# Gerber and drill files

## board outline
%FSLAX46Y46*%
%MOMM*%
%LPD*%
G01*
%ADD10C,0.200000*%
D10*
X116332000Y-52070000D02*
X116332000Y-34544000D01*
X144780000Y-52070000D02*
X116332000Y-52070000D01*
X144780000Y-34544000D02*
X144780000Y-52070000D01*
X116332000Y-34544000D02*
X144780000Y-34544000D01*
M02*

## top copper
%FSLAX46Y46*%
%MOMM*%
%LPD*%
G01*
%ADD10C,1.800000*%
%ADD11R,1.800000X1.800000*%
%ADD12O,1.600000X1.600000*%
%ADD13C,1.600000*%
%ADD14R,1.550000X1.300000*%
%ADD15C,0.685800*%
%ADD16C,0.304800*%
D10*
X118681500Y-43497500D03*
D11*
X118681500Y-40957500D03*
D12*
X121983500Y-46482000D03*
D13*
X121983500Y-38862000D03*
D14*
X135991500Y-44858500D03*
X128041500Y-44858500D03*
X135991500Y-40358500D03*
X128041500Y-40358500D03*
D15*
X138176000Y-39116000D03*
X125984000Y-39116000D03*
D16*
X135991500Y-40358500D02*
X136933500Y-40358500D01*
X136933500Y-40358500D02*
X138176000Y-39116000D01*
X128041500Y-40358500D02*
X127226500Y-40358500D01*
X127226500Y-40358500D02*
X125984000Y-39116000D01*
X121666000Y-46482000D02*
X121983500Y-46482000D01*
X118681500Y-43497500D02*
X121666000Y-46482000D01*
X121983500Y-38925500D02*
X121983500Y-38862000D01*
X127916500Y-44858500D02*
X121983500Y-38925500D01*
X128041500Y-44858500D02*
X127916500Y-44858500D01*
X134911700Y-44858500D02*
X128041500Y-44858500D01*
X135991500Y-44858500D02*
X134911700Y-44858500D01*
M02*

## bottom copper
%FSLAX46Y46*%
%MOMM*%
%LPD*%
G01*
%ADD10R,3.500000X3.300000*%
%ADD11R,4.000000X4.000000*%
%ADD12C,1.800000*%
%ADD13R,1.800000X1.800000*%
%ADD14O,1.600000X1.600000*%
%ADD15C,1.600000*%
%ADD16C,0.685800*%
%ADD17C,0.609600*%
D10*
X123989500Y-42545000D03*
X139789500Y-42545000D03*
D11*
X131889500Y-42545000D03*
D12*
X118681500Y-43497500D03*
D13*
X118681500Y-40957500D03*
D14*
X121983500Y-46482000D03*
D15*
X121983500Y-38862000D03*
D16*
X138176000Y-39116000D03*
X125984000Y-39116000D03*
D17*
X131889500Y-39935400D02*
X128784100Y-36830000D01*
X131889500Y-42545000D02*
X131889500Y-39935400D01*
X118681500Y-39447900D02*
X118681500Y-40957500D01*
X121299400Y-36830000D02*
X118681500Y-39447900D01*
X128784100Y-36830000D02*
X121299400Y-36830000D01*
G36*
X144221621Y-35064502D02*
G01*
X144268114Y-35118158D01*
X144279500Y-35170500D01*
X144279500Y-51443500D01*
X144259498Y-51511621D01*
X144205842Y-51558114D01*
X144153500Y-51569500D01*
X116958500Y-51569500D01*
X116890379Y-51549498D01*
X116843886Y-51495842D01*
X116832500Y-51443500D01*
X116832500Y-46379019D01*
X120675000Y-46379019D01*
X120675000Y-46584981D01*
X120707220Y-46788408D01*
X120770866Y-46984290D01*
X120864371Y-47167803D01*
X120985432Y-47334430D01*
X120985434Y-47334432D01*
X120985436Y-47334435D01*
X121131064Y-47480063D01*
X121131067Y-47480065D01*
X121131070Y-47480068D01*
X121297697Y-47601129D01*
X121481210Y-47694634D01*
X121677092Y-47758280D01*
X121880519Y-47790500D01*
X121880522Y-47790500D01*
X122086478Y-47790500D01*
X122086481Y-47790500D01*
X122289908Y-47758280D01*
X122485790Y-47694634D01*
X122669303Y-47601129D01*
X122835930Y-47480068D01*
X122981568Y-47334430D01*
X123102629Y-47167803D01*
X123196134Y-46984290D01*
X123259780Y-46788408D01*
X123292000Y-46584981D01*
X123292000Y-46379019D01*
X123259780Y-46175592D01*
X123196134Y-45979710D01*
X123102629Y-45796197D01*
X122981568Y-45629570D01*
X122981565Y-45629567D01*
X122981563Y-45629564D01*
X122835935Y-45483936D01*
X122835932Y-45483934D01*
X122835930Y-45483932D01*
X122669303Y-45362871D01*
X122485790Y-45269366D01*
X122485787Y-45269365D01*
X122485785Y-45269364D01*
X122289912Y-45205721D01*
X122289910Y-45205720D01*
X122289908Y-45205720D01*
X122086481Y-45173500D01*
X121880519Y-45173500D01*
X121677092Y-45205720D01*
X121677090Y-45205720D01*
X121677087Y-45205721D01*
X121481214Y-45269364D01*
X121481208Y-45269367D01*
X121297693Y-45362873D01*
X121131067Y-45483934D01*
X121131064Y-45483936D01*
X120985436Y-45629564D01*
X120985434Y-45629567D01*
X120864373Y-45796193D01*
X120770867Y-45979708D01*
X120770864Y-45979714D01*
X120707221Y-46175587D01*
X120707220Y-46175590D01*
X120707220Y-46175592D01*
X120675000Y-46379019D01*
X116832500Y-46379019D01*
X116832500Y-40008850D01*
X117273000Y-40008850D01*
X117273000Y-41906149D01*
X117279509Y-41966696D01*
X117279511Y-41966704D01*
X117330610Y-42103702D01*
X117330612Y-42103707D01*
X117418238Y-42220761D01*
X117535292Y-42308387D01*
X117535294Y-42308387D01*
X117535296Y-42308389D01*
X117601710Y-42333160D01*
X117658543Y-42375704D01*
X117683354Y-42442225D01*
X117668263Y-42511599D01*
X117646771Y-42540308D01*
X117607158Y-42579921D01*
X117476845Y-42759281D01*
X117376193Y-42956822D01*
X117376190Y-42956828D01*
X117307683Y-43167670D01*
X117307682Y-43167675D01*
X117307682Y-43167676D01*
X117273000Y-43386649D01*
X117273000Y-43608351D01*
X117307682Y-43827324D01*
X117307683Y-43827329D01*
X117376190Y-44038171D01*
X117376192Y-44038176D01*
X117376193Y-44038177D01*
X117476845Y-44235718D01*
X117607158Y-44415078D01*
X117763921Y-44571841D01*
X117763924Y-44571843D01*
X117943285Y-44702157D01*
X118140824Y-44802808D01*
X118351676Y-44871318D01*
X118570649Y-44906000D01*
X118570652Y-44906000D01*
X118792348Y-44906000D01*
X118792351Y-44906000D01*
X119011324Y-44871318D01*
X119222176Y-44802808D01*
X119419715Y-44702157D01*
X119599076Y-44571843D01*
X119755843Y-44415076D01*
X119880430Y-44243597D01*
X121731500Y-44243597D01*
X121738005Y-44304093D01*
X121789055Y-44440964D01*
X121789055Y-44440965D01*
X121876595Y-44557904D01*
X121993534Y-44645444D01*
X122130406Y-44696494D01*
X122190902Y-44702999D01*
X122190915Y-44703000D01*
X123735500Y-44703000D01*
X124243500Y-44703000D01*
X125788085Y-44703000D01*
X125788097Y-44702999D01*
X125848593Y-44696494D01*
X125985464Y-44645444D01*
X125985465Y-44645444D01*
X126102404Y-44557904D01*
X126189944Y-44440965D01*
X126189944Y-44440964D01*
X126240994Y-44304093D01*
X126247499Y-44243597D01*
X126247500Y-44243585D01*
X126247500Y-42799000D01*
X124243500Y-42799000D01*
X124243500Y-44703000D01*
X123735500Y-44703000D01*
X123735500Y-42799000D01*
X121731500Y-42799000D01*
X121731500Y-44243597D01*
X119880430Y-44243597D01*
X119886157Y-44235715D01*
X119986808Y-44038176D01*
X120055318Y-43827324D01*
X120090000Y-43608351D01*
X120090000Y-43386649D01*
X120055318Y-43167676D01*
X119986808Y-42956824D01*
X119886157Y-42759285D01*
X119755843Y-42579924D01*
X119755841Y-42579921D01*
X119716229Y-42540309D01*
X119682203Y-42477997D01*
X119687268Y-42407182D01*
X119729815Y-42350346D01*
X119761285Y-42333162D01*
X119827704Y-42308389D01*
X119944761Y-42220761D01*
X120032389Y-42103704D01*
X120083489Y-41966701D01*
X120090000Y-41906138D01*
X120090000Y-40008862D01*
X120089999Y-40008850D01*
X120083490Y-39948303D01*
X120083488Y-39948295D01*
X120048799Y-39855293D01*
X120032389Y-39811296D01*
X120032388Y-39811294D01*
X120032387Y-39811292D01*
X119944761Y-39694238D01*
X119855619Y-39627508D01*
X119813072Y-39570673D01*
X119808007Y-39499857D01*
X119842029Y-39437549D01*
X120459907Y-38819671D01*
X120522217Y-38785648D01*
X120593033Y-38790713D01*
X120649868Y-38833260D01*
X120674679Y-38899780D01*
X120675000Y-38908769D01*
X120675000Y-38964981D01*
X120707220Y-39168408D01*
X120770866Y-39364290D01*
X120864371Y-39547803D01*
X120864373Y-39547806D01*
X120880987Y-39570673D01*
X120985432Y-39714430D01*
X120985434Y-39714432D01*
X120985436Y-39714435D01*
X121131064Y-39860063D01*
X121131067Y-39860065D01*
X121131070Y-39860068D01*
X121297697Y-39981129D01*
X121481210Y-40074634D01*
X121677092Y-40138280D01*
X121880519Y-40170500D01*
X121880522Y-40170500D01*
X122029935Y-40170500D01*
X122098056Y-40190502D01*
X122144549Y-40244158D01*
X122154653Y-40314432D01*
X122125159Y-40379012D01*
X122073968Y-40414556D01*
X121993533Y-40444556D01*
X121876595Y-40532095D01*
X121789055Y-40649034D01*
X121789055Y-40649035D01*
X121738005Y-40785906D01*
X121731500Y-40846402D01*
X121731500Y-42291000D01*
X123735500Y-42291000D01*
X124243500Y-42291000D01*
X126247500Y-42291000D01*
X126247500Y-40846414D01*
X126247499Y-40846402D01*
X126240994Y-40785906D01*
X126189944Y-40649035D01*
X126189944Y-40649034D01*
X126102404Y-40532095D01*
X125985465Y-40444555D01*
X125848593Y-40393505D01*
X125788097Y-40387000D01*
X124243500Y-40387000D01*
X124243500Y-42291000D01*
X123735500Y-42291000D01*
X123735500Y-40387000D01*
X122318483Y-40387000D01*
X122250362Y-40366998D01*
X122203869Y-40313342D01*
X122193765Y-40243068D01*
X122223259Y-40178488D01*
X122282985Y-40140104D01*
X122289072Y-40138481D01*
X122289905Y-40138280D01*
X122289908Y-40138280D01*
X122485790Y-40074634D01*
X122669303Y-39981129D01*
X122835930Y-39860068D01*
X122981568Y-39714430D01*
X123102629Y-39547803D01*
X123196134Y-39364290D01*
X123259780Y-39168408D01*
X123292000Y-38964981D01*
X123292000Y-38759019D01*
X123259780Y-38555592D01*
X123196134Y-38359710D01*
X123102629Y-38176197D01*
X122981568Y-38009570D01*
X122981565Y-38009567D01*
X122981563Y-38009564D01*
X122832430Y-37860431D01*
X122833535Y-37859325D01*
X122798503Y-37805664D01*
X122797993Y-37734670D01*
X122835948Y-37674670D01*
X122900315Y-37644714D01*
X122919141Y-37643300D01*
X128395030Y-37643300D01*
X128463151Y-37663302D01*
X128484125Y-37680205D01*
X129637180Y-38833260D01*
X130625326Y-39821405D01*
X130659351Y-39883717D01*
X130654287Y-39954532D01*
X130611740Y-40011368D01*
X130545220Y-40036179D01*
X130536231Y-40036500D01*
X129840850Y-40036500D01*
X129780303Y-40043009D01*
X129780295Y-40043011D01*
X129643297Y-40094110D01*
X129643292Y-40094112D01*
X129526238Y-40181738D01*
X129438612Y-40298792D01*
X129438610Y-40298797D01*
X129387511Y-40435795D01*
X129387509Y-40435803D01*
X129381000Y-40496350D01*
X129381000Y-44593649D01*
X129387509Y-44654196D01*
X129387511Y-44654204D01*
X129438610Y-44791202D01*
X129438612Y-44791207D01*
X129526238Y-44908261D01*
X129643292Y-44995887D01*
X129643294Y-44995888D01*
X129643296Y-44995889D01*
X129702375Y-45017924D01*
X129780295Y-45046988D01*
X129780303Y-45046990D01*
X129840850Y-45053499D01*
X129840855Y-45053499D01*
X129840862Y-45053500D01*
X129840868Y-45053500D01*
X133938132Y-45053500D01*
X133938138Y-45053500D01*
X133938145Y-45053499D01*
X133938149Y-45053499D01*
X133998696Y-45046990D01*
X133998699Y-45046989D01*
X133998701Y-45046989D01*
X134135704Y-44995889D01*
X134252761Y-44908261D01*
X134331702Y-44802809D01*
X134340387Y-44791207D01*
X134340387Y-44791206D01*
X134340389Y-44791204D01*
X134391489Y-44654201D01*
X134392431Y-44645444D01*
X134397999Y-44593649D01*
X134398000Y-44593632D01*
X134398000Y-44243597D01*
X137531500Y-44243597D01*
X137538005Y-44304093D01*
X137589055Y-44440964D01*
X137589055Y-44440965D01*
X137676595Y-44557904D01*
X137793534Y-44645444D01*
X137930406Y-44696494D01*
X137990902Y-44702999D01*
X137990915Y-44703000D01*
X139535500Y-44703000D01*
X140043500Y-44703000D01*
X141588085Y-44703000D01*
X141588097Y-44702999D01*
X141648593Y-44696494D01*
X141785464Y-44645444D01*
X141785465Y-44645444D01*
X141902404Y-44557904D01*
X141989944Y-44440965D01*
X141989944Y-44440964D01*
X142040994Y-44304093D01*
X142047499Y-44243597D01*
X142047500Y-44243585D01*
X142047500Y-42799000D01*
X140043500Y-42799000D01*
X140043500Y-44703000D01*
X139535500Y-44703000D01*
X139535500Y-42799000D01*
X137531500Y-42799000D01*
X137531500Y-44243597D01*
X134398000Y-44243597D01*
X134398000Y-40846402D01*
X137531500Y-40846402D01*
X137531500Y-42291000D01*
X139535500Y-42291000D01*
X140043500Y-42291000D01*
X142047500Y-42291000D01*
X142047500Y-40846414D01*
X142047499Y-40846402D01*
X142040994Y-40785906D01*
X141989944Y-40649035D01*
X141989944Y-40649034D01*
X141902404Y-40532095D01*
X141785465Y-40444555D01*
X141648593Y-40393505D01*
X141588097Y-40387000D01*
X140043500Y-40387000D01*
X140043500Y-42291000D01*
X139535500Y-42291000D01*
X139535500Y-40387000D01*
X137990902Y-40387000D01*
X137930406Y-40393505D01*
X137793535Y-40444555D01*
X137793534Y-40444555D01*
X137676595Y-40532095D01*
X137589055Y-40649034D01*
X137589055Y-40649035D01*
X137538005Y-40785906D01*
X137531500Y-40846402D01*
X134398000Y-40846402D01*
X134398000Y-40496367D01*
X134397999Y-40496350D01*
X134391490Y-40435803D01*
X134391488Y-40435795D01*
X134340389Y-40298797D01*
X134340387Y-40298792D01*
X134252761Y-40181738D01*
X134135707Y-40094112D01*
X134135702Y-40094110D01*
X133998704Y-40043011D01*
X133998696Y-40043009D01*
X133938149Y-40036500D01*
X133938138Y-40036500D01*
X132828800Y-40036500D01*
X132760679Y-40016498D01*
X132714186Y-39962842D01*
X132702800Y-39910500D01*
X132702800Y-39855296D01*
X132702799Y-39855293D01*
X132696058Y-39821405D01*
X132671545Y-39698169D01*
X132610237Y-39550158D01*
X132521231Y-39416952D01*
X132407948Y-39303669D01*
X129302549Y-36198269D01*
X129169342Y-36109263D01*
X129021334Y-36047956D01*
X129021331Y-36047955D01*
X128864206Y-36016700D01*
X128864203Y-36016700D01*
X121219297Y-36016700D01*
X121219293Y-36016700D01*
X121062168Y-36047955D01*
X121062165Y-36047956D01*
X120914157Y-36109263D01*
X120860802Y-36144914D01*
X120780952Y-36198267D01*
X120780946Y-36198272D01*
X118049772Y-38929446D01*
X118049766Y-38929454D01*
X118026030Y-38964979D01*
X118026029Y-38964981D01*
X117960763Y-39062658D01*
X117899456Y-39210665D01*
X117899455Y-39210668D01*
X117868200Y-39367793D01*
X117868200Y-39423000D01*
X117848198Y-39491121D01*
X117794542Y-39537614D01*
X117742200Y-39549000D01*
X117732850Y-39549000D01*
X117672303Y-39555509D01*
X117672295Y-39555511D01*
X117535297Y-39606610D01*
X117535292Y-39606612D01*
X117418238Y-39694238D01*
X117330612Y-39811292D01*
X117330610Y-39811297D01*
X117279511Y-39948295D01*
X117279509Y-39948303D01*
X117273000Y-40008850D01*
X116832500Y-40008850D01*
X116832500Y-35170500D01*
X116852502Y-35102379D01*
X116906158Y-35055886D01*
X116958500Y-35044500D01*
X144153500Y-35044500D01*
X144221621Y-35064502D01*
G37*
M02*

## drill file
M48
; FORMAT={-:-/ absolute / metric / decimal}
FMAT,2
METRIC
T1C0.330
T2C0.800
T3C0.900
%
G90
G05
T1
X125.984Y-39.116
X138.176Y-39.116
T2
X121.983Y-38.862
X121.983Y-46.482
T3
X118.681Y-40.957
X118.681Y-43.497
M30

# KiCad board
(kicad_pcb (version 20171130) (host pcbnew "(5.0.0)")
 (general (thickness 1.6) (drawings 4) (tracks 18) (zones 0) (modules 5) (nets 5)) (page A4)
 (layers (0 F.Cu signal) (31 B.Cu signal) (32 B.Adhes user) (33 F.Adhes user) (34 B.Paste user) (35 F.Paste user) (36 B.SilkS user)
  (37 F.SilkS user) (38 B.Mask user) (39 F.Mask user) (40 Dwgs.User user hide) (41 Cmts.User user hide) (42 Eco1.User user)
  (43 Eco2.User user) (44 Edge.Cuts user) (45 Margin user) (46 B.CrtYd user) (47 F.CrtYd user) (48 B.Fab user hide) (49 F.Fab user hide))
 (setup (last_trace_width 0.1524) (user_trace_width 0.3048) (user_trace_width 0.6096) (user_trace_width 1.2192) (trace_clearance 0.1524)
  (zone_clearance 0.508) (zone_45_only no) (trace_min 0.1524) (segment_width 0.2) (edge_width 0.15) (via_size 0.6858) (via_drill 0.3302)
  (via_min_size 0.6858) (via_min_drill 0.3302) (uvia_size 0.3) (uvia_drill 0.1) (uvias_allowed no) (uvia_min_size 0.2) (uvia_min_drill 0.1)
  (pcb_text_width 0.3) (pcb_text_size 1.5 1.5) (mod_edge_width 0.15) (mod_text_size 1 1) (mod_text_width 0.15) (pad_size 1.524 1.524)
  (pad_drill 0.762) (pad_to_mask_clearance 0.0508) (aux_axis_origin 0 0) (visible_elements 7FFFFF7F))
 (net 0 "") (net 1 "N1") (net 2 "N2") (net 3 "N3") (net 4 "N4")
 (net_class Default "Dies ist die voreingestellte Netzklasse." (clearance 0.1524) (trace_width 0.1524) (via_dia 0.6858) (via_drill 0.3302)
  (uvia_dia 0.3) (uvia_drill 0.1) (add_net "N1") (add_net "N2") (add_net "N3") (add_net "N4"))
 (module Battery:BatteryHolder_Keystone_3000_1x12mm (layer B.Cu) (at 131.8895 42.545)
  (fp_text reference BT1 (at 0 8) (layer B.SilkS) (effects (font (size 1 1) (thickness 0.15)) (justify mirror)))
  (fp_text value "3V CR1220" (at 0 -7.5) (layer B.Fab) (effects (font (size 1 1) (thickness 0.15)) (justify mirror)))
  (pad 1 smd rect (at -7.9 0) (size 3.5 3.3) (layers B.Cu B.Paste B.Mask) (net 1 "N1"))
  (pad 1 smd rect (at 7.9 0) (size 3.5 3.3) (layers B.Cu B.Paste B.Mask) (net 1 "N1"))
  (pad 2 smd rect (at 0 0) (size 4 4) (layers B.Cu B.Mask) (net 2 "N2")))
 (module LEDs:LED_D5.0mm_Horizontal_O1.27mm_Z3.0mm (layer F.Cu) (at 118.6815 40.9575 270)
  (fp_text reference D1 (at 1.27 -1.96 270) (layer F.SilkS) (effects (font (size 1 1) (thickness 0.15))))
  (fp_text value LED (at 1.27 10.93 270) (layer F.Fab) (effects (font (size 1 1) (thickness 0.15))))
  (pad 2 thru_hole circle (at 2.54 0 270) (size 1.8 1.8) (drill 0.9) (layers *.Cu *.Mask) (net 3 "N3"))
  (pad 1 thru_hole rect (at 0 0 270) (size 1.8 1.8) (drill 0.9) (layers *.Cu *.Mask) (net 2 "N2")))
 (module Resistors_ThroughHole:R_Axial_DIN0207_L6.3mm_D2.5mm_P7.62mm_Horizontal (layer F.Cu) (at 121.9835 38.862 270)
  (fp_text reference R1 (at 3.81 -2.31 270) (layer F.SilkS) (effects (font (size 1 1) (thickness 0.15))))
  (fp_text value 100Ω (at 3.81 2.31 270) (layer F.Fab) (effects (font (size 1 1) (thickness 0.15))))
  (pad 2 thru_hole oval (at 7.62 0 270) (size 1.6 1.6) (drill 0.8) (layers *.Cu *.Mask) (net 3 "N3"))
  (pad 1 thru_hole circle (at 0 0 270) (size 1.6 1.6) (drill 0.8) (layers *.Cu *.Mask) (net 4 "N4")))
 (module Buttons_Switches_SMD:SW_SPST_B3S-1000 (layer F.Cu) (at 132.0165 42.6085)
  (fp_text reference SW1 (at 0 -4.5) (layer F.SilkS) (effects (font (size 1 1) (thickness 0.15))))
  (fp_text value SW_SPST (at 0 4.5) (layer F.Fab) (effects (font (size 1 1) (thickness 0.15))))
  (pad 2 smd rect (at 3.975 2.25) (size 1.55 1.3) (layers F.Cu F.Paste F.Mask) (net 4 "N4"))
  (pad 2 smd rect (at -3.975 2.25) (size 1.55 1.3) (layers F.Cu F.Paste F.Mask) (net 4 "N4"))
  (pad 1 smd rect (at 3.975 -2.25) (size 1.55 1.3) (layers F.Cu F.Paste F.Mask) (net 1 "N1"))
  (pad 1 smd rect (at -3.975 -2.25) (size 1.55 1.3) (layers F.Cu F.Paste F.Mask) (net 1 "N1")))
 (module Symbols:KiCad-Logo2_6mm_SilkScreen (layer F.Cu) (at 140.97 43.434 90)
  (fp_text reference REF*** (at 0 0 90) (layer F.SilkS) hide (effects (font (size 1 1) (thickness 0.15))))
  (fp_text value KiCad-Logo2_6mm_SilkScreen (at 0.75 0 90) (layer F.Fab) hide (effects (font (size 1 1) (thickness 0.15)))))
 (gr_line (start 116.332 52.07) (end 116.332 34.544) (layer Edge.Cuts) (width 0.2))
 (gr_line (start 144.78 52.07) (end 116.332 52.07) (layer Edge.Cuts) (width 0.2))
 (gr_line (start 144.78 34.544) (end 144.78 52.07) (layer Edge.Cuts) (width 0.2))
 (gr_line (start 116.332 34.544) (end 144.78 34.544) (layer Edge.Cuts) (width 0.2))
 (via (at 138.176 39.116) (size 0.6858) (drill 0.3302) (layers F.Cu B.Cu) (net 1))
 (segment (start 135.9915 40.3585) (end 136.9335 40.3585) (width 0.3048) (layer F.Cu) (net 1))
 (segment (start 136.9335 40.3585) (end 138.176 39.116) (width 0.3048) (layer F.Cu) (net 1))
 (via (at 125.984 39.116) (size 0.6858) (drill 0.3302) (layers F.Cu B.Cu) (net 1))
 (segment (start 128.0415 40.3585) (end 127.2265 40.3585) (width 0.3048) (layer F.Cu) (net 1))
 (segment (start 127.2265 40.3585) (end 125.984 39.116) (width 0.3048) (layer F.Cu) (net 1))
 (segment (start 131.8895 39.9354) (end 128.7841 36.83) (width 0.6096) (layer B.Cu) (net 2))
 (segment (start 131.8895 42.545) (end 131.8895 39.9354) (width 0.6096) (layer B.Cu) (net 2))
 (segment (start 118.6815 39.4479) (end 118.6815 40.9575) (width 0.6096) (layer B.Cu) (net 2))
 (segment (start 121.2994 36.83) (end 118.6815 39.4479) (width 0.6096) (layer B.Cu) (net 2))
 (segment (start 128.7841 36.83) (end 121.2994 36.83) (width 0.6096) (layer B.Cu) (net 2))
 (segment (start 121.666 46.482) (end 121.9835 46.482) (width 0.3048) (layer F.Cu) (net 3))
 (segment (start 118.6815 43.4975) (end 121.666 46.482) (width 0.3048) (layer F.Cu) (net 3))
 (segment (start 121.9835 38.9255) (end 121.9835 38.862) (width 0.3048) (layer F.Cu) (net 4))
 (segment (start 127.9165 44.8585) (end 121.9835 38.9255) (width 0.3048) (layer F.Cu) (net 4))
 (segment (start 128.0415 44.8585) (end 127.9165 44.8585) (width 0.3048) (layer F.Cu) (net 4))
 (segment (start 134.9117 44.8585) (end 128.0415 44.8585) (width 0.3048) (layer F.Cu) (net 4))
 (segment (start 135.9915 44.8585) (end 134.9117 44.8585) (width 0.3048) (layer F.Cu) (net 4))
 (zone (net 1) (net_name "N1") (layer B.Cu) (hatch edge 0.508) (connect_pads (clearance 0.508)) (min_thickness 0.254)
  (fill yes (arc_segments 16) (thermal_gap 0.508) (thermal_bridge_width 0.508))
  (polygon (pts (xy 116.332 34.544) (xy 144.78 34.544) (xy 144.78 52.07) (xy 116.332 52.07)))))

